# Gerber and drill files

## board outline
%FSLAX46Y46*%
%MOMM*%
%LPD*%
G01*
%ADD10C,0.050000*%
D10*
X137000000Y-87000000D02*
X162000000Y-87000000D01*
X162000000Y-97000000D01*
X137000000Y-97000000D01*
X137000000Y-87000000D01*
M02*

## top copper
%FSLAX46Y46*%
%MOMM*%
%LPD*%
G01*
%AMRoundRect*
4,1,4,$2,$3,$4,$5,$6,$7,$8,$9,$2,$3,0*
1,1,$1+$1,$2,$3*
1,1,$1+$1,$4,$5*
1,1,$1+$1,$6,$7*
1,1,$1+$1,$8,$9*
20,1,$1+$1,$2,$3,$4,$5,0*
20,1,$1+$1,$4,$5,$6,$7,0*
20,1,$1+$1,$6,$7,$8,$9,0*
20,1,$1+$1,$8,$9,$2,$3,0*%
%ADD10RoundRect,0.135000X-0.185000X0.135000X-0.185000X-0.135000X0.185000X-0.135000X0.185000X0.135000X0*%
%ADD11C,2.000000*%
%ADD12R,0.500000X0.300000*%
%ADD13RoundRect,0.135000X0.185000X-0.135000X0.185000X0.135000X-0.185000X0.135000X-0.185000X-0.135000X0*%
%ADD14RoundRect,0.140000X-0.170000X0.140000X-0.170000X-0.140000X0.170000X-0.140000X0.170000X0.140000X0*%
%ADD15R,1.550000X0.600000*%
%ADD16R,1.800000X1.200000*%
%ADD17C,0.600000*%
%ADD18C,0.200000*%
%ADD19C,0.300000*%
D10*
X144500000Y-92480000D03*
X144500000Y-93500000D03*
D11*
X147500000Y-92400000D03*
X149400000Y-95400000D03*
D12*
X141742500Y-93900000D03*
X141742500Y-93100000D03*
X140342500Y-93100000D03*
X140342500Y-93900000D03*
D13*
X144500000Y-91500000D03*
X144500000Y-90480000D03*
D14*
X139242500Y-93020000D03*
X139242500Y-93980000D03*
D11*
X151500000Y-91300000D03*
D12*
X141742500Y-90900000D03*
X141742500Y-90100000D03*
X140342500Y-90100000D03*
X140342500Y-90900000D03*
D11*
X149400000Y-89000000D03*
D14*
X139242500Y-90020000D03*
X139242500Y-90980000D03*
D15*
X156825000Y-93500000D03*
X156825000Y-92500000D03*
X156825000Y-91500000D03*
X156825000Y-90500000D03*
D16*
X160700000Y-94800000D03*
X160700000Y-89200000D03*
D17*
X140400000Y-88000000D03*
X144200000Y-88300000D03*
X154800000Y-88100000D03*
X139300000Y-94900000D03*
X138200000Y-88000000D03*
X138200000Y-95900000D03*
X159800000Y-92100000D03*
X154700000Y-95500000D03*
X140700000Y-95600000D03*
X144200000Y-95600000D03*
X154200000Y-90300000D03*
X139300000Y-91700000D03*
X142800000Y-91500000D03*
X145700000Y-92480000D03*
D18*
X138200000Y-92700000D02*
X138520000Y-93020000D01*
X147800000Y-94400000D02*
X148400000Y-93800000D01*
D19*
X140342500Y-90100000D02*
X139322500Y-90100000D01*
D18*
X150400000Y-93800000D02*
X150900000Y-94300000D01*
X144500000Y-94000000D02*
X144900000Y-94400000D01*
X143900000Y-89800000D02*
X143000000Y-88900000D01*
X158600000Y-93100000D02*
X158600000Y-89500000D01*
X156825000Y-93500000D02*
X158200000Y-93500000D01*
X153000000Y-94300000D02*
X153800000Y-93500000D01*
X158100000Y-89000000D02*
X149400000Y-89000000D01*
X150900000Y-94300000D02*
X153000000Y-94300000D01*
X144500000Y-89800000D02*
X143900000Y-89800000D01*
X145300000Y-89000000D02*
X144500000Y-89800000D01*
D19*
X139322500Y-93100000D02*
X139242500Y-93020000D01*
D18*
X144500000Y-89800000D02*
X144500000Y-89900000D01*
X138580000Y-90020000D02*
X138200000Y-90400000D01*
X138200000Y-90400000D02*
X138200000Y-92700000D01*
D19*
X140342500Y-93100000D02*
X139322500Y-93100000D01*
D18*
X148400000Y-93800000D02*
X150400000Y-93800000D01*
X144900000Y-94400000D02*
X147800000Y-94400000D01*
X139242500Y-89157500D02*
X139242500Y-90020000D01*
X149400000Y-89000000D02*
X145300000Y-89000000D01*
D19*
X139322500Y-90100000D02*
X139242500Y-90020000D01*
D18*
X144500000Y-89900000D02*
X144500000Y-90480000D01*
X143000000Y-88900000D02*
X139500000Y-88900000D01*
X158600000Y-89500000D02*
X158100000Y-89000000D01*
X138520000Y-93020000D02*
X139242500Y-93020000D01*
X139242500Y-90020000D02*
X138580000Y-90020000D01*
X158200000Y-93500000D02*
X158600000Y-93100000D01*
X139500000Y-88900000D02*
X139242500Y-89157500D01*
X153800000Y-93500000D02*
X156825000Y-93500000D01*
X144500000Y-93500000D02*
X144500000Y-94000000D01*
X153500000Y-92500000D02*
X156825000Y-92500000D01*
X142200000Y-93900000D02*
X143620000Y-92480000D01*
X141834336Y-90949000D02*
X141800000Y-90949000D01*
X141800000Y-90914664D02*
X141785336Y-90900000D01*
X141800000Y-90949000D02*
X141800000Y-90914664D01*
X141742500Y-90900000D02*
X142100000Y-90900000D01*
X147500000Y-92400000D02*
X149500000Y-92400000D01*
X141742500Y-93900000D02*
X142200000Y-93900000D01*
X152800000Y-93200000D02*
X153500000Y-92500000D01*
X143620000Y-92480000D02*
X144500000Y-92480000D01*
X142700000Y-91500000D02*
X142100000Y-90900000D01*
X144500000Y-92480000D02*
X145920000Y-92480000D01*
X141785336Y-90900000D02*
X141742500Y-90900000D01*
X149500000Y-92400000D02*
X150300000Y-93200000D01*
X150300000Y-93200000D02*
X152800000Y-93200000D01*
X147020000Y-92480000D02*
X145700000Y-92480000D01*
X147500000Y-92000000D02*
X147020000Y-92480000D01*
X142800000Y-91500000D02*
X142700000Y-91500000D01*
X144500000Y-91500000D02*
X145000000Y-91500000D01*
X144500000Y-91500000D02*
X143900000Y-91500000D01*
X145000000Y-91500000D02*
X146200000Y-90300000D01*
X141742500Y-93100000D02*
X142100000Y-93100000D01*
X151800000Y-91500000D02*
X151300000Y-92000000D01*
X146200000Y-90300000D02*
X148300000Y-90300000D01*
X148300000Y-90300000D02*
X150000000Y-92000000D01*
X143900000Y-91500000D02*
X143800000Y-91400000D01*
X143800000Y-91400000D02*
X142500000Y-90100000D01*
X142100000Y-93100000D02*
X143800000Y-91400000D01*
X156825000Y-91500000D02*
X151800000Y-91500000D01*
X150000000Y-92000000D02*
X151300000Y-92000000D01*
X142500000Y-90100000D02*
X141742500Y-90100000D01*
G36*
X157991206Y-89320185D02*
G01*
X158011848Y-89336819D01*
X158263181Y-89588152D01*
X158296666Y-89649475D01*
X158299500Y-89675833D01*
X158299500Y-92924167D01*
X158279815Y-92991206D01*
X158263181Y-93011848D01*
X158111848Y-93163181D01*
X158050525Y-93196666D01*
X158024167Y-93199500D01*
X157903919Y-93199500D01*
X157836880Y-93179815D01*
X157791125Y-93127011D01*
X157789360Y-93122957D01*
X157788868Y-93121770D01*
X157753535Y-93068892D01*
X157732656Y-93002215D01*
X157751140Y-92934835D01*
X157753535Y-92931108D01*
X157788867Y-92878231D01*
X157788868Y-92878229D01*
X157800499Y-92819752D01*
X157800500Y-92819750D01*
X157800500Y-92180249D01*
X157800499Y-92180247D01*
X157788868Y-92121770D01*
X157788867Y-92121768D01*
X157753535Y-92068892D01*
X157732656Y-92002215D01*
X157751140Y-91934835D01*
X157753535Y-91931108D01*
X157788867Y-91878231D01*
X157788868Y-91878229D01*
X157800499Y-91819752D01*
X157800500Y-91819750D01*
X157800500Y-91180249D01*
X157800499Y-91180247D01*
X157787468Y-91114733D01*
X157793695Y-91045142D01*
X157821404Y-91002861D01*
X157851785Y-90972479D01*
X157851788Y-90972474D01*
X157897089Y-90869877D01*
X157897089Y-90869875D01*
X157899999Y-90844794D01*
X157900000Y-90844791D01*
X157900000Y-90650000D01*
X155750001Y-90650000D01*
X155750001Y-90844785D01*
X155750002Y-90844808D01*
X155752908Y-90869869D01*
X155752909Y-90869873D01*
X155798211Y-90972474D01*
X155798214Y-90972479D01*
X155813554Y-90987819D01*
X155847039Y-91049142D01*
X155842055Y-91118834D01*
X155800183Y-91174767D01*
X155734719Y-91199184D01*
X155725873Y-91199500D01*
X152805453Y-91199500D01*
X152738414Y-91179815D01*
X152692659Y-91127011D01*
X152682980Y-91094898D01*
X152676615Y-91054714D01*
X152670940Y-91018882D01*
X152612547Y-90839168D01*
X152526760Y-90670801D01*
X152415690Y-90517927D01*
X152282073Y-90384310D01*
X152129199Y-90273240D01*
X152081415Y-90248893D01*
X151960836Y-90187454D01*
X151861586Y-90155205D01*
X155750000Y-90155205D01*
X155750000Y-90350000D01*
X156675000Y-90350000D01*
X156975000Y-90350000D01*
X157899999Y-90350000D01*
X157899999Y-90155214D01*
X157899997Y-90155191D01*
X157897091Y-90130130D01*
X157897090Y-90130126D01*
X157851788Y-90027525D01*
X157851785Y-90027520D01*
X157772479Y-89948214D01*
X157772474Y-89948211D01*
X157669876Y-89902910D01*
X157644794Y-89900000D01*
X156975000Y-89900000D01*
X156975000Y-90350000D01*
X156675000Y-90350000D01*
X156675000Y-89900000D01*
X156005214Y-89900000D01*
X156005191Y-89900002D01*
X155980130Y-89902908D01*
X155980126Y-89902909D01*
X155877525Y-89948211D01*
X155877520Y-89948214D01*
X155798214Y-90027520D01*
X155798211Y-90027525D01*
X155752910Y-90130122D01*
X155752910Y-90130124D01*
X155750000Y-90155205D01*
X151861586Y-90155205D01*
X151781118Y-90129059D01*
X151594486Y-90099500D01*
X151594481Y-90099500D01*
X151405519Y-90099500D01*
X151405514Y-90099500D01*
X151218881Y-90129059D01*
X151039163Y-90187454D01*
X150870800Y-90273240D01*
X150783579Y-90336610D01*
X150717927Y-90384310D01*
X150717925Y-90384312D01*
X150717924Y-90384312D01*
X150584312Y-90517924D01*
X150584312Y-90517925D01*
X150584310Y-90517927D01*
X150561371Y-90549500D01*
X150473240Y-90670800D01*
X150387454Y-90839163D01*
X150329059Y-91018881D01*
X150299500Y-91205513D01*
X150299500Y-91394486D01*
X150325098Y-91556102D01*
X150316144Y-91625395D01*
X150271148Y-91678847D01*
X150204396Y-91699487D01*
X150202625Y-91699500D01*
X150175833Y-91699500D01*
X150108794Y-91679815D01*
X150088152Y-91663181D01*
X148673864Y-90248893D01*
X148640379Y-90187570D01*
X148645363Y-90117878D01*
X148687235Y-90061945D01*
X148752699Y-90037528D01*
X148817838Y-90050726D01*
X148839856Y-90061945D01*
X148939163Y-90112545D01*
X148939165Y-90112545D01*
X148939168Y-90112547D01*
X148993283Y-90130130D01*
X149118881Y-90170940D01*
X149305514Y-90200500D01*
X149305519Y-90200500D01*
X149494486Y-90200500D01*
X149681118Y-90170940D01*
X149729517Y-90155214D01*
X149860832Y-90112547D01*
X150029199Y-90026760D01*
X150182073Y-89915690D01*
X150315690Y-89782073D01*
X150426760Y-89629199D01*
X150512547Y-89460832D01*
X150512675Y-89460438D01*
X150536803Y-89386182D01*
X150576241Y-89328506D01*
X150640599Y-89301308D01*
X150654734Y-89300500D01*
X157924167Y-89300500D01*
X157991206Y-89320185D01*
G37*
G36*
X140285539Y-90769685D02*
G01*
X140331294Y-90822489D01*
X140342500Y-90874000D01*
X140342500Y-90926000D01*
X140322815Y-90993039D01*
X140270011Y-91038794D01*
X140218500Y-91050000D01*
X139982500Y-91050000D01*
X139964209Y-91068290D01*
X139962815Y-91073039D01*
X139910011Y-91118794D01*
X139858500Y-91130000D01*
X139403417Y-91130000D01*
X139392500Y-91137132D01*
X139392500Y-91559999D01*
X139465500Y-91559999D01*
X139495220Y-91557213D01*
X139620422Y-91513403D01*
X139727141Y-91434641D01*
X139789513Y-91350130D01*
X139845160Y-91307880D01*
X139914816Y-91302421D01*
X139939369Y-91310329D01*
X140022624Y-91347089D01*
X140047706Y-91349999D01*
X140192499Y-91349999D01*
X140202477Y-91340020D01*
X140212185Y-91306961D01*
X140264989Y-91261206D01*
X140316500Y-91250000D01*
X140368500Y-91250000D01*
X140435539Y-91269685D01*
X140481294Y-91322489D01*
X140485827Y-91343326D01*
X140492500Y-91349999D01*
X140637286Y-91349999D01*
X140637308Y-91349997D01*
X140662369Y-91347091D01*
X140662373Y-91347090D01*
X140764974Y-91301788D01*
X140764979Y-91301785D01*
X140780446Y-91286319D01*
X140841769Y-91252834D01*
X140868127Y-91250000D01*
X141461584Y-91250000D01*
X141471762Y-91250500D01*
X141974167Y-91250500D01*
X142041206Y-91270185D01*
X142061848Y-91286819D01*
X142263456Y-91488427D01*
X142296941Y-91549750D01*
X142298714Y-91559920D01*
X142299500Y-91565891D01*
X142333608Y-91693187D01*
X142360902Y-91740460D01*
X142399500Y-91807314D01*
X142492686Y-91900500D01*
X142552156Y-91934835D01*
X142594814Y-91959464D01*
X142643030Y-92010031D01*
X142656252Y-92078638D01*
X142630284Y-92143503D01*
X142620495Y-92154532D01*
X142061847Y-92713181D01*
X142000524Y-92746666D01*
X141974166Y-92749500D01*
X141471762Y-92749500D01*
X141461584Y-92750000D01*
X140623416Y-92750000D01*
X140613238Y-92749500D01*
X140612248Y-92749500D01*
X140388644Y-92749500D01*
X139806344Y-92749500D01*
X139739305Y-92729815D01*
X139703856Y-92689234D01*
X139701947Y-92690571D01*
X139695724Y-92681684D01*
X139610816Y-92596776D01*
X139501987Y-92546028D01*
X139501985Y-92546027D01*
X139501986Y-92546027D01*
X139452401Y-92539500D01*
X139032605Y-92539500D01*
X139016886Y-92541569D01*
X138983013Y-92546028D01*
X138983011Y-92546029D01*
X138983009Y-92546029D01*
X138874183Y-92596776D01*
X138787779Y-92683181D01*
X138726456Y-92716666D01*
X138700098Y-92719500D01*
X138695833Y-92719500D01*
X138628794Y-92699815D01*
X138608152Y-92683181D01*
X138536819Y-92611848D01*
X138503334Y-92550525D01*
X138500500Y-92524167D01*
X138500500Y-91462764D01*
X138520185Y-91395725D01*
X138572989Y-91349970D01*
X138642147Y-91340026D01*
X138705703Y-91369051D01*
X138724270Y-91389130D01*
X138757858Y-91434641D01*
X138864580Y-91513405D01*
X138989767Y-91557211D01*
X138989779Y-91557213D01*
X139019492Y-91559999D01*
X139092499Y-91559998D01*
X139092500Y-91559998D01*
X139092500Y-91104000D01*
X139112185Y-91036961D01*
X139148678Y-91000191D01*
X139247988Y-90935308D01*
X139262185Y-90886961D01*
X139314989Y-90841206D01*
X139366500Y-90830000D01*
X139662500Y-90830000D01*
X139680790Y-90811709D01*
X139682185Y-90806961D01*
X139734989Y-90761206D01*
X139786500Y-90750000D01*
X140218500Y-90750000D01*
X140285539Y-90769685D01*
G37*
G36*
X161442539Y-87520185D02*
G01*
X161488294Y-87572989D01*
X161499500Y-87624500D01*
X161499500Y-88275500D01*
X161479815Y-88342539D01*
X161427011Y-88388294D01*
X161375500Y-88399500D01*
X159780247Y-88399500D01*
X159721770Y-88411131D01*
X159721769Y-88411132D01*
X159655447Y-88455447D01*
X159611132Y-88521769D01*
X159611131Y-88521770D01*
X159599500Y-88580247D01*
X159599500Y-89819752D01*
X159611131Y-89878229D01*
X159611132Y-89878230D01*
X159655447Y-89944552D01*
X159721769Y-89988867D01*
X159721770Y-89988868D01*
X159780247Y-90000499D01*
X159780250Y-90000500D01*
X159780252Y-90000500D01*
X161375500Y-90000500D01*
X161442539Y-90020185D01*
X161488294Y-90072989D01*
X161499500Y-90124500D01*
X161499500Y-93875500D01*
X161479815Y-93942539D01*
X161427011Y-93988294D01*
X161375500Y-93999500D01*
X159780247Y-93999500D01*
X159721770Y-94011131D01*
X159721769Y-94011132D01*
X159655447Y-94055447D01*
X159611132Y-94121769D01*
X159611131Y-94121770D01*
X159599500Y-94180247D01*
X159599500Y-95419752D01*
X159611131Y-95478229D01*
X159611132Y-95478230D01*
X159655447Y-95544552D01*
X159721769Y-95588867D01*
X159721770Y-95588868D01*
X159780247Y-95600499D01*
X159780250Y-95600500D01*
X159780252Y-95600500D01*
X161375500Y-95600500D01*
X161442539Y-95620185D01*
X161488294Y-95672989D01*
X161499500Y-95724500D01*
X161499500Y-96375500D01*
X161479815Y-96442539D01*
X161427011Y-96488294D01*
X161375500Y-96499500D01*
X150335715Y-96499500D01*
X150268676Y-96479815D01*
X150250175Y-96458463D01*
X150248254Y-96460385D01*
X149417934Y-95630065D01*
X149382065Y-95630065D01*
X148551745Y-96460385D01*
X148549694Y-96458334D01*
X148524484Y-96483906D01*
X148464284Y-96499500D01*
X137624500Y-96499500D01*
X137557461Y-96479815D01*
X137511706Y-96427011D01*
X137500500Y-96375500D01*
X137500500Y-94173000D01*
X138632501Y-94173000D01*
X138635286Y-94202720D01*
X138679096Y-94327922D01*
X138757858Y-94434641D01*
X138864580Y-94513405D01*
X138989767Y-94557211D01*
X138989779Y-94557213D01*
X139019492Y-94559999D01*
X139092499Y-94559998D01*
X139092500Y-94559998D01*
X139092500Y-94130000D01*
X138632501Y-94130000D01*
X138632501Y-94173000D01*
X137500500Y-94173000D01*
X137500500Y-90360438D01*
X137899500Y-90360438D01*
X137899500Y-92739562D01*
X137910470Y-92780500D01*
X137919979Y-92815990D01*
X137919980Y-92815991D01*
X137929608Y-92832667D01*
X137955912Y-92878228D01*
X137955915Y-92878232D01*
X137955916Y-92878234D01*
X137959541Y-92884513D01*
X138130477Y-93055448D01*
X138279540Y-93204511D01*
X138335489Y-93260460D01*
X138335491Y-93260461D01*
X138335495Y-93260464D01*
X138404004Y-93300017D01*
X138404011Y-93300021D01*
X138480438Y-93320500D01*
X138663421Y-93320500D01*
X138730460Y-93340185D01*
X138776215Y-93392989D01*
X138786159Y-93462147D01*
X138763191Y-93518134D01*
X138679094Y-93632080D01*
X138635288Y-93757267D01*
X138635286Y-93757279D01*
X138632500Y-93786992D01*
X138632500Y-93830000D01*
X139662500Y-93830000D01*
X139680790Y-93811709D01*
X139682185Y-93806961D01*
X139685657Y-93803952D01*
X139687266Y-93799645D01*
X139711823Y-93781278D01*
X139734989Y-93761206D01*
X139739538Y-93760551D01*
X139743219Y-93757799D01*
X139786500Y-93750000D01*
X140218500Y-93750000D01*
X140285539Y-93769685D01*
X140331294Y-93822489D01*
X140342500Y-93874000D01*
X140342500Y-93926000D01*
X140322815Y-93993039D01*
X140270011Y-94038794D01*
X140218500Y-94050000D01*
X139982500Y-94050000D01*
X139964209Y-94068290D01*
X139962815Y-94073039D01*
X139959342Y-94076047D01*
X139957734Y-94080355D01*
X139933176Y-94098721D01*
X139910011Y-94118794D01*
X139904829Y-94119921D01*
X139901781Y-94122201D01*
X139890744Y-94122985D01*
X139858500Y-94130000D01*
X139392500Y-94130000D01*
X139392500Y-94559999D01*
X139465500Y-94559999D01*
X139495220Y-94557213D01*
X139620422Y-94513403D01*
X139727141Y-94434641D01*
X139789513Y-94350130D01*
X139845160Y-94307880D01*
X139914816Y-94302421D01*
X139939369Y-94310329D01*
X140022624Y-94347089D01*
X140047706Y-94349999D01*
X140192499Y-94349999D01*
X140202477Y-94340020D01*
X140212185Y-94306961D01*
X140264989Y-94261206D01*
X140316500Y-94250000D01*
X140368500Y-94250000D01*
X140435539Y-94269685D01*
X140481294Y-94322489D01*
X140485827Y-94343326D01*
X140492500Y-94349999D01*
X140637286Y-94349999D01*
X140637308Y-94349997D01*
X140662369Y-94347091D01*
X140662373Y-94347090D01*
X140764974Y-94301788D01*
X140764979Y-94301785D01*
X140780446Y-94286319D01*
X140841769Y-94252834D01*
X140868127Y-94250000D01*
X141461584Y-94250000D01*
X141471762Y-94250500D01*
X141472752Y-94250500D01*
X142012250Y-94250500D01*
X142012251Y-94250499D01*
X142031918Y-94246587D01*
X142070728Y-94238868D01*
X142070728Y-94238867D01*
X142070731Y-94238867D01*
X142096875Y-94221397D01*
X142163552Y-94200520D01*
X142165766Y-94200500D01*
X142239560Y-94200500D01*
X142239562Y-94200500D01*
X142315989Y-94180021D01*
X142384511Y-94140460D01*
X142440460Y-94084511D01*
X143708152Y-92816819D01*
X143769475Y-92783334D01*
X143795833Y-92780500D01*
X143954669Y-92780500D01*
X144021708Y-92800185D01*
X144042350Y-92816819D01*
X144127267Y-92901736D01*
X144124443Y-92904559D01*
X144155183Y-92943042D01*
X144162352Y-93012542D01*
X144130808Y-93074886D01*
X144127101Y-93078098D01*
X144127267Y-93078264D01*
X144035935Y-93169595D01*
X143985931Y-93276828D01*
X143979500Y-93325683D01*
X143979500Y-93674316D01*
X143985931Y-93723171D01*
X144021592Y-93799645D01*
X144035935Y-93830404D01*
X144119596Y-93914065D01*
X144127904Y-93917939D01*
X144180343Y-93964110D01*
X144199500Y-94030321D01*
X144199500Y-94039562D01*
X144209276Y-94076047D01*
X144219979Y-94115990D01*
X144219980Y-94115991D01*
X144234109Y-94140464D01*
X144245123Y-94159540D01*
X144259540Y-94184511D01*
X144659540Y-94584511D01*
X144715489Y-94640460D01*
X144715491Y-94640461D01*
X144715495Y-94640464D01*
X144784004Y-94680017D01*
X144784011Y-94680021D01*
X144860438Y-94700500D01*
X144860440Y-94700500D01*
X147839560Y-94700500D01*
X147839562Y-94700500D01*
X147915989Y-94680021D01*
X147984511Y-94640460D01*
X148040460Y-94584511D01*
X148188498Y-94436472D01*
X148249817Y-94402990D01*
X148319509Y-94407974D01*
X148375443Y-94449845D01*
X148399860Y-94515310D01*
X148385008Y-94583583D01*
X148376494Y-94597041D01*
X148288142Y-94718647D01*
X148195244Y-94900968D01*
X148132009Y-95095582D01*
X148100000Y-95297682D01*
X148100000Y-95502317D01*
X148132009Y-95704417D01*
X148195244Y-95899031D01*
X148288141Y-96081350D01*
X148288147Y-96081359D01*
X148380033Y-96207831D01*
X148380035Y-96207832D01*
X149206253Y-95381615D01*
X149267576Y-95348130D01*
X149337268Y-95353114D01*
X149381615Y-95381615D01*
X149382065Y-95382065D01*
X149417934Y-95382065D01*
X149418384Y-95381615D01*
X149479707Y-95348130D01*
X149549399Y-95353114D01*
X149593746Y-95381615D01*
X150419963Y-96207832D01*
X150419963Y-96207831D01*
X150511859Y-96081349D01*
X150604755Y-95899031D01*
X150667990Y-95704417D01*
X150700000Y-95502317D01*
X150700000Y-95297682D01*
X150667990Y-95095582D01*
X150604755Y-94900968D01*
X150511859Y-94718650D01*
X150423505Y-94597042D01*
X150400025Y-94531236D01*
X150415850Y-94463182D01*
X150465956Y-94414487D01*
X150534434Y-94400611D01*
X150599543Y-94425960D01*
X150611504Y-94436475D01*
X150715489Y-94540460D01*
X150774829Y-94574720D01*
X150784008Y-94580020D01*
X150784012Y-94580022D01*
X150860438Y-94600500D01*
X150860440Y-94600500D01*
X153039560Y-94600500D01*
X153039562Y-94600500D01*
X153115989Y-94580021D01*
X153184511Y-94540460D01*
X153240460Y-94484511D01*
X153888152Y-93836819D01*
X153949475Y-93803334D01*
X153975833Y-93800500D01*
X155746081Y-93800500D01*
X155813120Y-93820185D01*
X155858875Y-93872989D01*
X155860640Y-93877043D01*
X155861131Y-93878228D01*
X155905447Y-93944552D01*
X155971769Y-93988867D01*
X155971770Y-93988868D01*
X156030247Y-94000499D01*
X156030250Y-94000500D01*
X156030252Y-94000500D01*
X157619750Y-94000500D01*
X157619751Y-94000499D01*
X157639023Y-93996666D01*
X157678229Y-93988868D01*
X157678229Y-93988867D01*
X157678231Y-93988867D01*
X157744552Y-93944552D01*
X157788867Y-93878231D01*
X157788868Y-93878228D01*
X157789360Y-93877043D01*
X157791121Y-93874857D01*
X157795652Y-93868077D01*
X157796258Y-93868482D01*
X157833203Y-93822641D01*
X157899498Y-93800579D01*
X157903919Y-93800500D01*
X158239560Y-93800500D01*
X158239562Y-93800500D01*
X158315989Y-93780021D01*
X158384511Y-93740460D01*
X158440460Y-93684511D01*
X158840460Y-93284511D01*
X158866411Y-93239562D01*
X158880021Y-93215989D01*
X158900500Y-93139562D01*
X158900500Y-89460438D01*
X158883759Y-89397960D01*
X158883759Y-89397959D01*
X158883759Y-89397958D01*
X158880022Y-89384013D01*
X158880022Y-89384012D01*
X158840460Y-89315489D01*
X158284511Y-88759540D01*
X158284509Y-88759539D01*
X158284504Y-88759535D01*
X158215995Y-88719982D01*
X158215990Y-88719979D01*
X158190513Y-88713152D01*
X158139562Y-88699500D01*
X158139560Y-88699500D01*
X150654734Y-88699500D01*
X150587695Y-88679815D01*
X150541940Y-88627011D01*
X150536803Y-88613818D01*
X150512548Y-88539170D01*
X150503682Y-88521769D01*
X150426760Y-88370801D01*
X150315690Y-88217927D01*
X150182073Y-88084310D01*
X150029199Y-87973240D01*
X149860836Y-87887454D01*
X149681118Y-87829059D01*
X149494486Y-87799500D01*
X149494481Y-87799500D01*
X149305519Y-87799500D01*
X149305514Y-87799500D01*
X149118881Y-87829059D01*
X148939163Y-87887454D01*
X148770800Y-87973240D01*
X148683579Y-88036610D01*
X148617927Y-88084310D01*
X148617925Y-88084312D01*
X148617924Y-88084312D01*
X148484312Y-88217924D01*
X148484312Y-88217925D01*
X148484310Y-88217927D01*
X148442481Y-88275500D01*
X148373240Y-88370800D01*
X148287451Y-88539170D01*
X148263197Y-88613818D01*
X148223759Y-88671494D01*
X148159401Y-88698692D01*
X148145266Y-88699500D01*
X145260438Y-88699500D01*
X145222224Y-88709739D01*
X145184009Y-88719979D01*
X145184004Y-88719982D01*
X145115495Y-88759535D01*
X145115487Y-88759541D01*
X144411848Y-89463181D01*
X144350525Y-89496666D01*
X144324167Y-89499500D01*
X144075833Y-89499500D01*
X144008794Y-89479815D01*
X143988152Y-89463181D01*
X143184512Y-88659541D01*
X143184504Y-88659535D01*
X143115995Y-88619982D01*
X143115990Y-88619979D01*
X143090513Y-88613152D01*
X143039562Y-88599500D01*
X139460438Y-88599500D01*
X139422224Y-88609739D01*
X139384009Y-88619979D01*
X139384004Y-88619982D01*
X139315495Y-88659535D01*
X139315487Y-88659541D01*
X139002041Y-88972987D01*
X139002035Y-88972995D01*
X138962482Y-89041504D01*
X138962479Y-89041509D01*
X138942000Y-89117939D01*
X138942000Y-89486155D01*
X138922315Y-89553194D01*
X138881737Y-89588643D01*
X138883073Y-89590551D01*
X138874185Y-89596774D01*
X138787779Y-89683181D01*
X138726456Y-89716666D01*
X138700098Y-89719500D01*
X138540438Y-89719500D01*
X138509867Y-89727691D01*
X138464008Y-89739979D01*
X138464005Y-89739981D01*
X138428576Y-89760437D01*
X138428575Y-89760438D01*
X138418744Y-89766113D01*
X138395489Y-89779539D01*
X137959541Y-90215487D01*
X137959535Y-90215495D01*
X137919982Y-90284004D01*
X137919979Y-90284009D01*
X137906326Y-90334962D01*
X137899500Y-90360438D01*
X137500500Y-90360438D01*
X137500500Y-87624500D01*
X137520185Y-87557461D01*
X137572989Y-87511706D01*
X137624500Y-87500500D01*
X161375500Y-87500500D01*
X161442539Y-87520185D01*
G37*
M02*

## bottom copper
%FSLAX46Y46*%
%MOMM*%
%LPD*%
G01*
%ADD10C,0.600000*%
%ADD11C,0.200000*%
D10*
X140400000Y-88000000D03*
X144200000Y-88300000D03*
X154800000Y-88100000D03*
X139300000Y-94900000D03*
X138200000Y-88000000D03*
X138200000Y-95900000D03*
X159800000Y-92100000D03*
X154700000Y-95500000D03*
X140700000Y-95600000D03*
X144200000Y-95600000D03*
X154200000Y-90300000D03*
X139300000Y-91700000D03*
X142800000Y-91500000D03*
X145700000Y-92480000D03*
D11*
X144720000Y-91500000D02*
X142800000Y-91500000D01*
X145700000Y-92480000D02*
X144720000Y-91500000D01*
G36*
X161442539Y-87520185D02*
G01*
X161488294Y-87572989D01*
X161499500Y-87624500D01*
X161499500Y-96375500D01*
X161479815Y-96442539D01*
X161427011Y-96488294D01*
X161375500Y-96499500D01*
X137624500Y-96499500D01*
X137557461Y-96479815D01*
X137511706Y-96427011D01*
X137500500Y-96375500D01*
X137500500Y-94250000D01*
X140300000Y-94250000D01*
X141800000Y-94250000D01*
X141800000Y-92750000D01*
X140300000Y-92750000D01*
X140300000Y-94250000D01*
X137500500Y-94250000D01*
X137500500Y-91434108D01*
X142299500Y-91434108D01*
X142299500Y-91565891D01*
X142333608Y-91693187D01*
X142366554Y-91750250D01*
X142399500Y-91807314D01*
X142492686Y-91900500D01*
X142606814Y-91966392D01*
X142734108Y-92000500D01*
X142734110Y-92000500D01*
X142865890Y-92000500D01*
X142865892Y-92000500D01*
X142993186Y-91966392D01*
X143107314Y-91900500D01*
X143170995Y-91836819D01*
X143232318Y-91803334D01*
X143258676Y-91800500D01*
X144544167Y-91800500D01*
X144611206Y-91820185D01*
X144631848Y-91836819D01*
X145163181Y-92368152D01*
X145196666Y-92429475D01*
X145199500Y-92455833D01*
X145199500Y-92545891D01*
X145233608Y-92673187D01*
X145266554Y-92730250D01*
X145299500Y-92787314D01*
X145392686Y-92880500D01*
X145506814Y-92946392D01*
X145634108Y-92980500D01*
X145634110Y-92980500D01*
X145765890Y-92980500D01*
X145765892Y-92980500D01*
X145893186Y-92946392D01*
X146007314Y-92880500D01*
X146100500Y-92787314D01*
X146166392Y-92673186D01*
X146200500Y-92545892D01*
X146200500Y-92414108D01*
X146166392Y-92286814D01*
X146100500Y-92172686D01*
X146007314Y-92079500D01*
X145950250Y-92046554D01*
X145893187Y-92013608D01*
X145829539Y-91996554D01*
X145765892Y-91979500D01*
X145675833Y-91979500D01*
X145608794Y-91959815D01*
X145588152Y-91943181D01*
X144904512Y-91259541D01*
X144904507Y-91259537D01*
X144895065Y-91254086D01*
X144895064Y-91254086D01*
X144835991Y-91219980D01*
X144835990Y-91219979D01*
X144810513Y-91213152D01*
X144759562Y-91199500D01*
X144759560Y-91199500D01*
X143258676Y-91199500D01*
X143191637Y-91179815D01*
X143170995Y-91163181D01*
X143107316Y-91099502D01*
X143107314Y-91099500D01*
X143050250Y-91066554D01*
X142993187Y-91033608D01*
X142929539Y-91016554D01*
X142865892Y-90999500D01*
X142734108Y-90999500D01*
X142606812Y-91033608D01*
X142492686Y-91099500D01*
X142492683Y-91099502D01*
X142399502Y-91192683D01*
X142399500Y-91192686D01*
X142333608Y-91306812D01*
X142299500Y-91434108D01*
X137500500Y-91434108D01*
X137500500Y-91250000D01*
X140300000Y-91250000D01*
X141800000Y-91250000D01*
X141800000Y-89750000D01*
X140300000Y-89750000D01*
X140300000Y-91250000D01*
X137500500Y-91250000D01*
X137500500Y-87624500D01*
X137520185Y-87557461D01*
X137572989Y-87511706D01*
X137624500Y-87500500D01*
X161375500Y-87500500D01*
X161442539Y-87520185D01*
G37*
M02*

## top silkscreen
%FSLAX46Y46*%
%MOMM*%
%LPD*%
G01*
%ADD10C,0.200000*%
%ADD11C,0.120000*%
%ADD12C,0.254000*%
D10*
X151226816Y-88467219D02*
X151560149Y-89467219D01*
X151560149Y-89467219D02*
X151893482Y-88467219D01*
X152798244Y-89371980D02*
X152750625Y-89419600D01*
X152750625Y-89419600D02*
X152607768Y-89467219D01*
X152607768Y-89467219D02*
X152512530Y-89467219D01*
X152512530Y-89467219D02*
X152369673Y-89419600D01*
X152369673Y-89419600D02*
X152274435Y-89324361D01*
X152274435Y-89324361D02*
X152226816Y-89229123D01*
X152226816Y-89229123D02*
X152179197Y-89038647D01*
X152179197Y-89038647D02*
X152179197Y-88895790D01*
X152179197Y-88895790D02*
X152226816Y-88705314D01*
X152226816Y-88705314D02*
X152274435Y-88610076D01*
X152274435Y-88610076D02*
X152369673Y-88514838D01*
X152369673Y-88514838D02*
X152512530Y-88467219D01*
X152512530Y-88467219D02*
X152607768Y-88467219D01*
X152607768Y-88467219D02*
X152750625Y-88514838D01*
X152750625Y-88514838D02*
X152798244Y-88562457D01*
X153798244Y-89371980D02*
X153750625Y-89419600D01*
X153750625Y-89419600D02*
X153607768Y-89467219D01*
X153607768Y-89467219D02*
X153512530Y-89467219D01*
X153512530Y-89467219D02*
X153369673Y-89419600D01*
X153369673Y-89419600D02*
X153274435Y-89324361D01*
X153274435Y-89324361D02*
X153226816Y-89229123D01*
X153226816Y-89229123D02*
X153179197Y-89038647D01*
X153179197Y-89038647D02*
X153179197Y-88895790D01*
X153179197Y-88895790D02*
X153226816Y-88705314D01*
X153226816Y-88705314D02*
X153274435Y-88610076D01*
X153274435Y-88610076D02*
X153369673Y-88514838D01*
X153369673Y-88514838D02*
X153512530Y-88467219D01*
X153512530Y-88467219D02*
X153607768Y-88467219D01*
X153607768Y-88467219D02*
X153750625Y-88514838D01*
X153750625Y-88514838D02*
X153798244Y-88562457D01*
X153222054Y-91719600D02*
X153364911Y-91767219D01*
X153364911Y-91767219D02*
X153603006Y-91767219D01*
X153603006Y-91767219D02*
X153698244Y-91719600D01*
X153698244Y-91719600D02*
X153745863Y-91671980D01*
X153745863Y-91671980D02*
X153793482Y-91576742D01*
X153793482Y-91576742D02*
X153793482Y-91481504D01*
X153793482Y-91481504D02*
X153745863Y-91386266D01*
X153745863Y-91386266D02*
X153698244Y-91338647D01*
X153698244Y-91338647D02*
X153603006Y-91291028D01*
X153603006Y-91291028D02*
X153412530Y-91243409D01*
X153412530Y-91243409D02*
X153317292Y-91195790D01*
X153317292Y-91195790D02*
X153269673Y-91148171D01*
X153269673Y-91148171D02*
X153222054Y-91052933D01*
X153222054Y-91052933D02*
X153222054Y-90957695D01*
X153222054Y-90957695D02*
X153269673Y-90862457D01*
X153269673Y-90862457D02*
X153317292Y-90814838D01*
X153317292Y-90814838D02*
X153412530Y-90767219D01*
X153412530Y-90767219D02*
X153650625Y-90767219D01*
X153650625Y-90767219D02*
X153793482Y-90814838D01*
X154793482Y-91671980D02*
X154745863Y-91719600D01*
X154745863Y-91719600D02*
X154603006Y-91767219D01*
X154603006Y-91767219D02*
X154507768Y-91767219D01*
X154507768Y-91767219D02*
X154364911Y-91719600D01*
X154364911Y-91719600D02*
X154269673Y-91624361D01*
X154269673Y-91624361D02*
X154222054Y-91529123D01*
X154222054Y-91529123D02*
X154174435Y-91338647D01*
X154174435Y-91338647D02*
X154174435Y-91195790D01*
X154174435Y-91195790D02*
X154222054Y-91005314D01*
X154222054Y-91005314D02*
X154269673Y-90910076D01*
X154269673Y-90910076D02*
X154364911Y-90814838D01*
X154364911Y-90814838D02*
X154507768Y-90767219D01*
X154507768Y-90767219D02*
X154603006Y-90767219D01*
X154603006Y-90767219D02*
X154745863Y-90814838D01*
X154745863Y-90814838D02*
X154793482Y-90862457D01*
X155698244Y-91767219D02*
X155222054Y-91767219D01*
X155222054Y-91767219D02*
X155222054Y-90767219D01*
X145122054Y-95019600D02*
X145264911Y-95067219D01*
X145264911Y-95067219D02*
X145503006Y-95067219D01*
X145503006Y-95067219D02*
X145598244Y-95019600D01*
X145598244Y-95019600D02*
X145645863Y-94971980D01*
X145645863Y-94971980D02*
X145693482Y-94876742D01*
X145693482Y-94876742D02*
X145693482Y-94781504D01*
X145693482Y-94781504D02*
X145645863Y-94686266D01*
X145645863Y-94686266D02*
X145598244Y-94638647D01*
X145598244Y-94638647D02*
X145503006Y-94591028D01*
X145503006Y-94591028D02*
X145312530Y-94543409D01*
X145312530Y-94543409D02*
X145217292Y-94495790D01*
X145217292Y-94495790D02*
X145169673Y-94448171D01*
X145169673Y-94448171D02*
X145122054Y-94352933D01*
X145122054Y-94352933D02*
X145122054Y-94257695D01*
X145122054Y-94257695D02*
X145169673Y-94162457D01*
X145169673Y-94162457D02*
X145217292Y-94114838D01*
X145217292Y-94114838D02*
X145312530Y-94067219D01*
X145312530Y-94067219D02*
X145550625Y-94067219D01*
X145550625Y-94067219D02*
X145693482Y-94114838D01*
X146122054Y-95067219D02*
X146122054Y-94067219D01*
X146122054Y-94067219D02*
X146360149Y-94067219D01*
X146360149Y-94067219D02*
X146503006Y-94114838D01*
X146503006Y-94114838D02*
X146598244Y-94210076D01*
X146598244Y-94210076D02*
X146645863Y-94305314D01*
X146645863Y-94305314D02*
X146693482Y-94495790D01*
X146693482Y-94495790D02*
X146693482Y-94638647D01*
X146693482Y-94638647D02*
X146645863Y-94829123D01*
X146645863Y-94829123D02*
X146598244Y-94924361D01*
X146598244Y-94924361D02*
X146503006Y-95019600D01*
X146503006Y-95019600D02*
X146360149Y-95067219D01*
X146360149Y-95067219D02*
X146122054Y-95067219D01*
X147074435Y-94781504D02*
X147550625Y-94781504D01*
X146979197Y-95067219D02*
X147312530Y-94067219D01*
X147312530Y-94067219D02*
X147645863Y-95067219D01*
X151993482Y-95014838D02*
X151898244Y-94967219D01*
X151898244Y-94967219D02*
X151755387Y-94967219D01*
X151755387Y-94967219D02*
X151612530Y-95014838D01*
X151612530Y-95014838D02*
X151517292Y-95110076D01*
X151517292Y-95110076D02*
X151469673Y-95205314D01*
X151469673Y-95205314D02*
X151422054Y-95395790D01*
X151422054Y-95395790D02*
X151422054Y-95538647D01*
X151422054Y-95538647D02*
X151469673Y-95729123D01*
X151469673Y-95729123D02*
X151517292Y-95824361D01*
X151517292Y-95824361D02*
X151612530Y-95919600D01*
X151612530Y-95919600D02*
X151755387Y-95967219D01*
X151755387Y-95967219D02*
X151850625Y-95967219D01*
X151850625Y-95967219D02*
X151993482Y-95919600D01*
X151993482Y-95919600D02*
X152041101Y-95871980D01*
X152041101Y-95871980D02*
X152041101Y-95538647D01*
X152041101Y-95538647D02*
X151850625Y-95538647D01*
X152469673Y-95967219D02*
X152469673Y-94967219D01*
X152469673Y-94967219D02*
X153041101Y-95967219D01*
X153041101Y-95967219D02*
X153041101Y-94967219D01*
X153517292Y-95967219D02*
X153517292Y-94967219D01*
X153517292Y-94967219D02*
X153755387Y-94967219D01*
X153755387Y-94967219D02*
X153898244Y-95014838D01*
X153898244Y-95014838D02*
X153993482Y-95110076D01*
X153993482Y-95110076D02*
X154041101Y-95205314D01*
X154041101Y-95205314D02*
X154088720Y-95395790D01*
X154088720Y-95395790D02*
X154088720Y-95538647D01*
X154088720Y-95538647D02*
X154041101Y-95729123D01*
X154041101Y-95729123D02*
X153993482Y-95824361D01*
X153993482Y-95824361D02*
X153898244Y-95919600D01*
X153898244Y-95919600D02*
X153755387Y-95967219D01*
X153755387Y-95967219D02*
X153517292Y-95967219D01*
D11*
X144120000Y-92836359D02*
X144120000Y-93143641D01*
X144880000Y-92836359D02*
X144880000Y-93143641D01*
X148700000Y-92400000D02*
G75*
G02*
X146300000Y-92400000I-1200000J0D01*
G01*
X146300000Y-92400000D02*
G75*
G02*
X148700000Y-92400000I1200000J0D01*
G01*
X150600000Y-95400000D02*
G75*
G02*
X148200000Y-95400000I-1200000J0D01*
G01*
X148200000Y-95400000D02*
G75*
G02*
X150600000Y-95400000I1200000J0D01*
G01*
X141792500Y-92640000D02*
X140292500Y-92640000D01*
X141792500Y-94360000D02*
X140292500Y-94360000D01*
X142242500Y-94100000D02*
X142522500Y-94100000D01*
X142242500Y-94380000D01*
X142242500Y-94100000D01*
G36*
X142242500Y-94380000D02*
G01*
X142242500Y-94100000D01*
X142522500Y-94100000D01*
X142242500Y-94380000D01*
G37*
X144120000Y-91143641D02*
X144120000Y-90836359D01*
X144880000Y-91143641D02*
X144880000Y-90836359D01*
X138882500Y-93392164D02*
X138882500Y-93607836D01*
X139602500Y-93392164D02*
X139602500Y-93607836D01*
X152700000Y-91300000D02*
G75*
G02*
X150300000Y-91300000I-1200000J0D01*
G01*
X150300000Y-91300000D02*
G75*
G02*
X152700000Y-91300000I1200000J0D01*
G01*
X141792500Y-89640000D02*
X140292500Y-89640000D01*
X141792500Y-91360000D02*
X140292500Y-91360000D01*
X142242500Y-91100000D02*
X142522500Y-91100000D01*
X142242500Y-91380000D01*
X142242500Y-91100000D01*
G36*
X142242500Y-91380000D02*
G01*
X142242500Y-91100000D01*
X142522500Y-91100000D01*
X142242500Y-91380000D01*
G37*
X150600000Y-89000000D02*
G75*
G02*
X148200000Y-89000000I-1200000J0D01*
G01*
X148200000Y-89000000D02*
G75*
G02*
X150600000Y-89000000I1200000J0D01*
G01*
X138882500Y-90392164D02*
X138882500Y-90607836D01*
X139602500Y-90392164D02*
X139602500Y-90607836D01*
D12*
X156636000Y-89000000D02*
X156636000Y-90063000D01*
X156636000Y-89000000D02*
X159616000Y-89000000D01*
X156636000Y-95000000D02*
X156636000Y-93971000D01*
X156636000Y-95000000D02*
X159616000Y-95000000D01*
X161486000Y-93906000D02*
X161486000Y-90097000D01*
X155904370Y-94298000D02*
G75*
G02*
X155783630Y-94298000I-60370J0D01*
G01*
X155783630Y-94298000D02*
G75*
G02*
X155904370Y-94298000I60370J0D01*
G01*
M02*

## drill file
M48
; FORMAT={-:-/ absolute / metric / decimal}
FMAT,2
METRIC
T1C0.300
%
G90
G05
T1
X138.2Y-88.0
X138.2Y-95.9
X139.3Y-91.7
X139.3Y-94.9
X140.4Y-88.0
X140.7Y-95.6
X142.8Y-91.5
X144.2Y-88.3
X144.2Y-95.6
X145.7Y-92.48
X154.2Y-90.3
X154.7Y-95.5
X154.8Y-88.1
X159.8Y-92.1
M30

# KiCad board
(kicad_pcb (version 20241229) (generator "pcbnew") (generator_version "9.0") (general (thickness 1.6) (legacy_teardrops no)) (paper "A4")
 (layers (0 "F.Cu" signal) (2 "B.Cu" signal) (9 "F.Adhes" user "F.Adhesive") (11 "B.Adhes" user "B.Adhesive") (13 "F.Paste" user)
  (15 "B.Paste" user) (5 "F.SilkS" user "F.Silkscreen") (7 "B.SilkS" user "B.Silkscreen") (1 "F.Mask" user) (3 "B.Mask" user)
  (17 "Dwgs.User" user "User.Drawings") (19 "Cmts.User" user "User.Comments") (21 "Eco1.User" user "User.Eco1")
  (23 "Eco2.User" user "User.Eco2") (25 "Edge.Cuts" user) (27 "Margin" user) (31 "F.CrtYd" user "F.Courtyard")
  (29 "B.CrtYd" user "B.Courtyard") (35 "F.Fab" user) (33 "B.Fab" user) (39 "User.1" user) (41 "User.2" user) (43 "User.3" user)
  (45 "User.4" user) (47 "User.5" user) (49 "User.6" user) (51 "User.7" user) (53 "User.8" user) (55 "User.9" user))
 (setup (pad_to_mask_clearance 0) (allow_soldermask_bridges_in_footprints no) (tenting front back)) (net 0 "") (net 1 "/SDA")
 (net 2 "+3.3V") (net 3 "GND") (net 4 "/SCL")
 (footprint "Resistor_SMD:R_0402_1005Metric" (layer "F.Cu") (at 144.5 92.99 -90)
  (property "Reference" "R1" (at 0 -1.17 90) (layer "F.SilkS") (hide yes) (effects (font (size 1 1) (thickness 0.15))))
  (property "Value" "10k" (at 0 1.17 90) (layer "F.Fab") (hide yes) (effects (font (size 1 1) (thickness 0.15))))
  (fp_line (start -0.153641 0.38) (end 0.153641 0.38) (stroke (width 0.12) (type solid)) (layer "F.SilkS"))
  (fp_line (start -0.153641 -0.38) (end 0.153641 -0.38) (stroke (width 0.12) (type solid)) (layer "F.SilkS"))
  (pad "1" smd roundrect (at -0.51 0 270) (size 0.54 0.64) (layers "F.Cu" "F.Mask" "F.Paste") (roundrect_rratio 0.25) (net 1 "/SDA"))
  (pad "2" smd roundrect (at 0.51 0 270) (size 0.54 0.64) (layers "F.Cu" "F.Mask" "F.Paste") (roundrect_rratio 0.25) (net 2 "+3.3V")))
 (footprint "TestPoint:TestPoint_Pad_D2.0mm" (layer "F.Cu") (at 147.5 92.4)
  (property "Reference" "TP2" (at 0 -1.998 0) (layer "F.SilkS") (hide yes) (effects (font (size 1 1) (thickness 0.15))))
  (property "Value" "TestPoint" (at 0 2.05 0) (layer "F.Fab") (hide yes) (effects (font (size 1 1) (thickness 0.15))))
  (fp_circle (center 0 0) (end 0 1.2) (stroke (width 0.12) (type solid)) (fill no) (layer "F.SilkS"))
  (pad "1" smd circle (at 0 0) (size 2 2) (layers "F.Cu" "F.Mask") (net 1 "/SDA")))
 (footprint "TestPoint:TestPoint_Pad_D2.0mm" (layer "F.Cu") (at 149.4 95.4)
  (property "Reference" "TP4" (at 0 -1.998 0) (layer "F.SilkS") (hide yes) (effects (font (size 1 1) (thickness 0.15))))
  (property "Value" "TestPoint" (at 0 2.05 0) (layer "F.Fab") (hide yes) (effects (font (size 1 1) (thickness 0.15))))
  (fp_circle (center 0 0) (end 0 1.2) (stroke (width 0.12) (type solid)) (fill no) (layer "F.SilkS"))
  (pad "1" smd circle (at 0 0) (size 2 2) (layers "F.Cu" "F.Mask") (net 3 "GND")))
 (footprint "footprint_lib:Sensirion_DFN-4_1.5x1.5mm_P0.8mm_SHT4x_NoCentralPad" (layer "F.Cu") (at 141.0425 93.5 180)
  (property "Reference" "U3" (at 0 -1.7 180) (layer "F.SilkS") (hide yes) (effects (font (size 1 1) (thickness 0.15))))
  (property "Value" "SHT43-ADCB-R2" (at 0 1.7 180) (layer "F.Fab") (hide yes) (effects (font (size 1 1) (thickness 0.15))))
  (fp_line (start -0.75 0.86) (end 0.75 0.86) (stroke (width 0.12) (type solid)) (layer "F.SilkS"))
  (fp_line (start -0.75 -0.86) (end 0.75 -0.86) (stroke (width 0.12) (type solid)) (layer "F.SilkS"))
  (fp_poly
   (pts (xy -1.2 -0.6) (xy -1.48 -0.6) (xy -1.2 -0.88) (xy -1.2 -0.6)) (stroke (width 0.12) (type solid)) (fill yes) (layer "F.SilkS"))
  (pad "1" smd rect (at -0.7 -0.4 180) (size 0.5 0.3) (layers "F.Cu" "F.Mask" "F.Paste") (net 1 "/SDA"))
  (pad "2" smd rect (at -0.7 0.4 180) (size 0.5 0.3) (layers "F.Cu" "F.Mask" "F.Paste") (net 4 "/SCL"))
  (pad "3" smd rect (at 0.7 0.4 180) (size 0.5 0.3) (layers "F.Cu" "F.Mask" "F.Paste") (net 2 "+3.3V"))
  (pad "4" smd rect (at 0.7 -0.4 180) (size 0.5 0.3) (layers "F.Cu" "F.Mask" "F.Paste") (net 3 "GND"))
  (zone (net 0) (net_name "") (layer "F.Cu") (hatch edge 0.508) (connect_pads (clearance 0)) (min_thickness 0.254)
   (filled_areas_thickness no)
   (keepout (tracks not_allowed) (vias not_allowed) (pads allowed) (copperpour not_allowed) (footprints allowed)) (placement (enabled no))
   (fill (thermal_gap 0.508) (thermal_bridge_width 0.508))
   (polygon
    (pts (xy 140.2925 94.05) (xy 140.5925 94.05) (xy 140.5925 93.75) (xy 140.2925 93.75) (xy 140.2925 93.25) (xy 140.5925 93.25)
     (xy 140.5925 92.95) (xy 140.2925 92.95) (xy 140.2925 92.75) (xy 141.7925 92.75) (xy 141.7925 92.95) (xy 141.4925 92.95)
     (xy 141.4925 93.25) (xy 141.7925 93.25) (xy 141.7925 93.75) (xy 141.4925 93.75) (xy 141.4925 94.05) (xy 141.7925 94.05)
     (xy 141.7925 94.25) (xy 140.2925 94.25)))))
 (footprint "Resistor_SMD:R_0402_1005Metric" (layer "F.Cu") (at 144.5 90.99 90)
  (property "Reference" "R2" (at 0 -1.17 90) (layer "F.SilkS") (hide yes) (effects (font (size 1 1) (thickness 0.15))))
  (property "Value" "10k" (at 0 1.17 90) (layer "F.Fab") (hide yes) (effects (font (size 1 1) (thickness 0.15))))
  (fp_line (start -0.153641 -0.38) (end 0.153641 -0.38) (stroke (width 0.12) (type solid)) (layer "F.SilkS"))
  (fp_line (start -0.153641 0.38) (end 0.153641 0.38) (stroke (width 0.12) (type solid)) (layer "F.SilkS"))
  (pad "1" smd roundrect (at -0.51 0 90) (size 0.54 0.64) (layers "F.Cu" "F.Mask" "F.Paste") (roundrect_rratio 0.25) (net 4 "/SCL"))
  (pad "2" smd roundrect (at 0.51 0 90) (size 0.54 0.64) (layers "F.Cu" "F.Mask" "F.Paste") (roundrect_rratio 0.25) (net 2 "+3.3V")))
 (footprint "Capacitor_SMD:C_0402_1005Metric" (layer "F.Cu") (at 139.2425 93.5 -90)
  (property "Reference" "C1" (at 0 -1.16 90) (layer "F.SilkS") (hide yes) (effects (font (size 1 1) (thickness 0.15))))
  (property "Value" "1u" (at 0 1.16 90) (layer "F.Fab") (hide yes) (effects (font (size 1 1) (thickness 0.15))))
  (fp_line (start -0.107836 0.36) (end 0.107836 0.36) (stroke (width 0.12) (type solid)) (layer "F.SilkS"))
  (fp_line (start -0.107836 -0.36) (end 0.107836 -0.36) (stroke (width 0.12) (type solid)) (layer "F.SilkS"))
  (pad "1" smd roundrect (at -0.48 0 270) (size 0.56 0.62) (layers "F.Cu" "F.Mask" "F.Paste") (roundrect_rratio 0.25) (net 2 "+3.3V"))
  (pad "2" smd roundrect (at 0.48 0 270) (size 0.56 0.62) (layers "F.Cu" "F.Mask" "F.Paste") (roundrect_rratio 0.25) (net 3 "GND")))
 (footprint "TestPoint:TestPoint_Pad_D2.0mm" (layer "F.Cu") (at 151.5 91.3)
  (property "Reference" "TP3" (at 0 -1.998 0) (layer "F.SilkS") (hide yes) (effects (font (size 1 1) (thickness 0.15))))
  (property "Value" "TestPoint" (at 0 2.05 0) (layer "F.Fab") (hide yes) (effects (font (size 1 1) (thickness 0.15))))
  (fp_circle (center 0 0) (end 0 1.2) (stroke (width 0.12) (type solid)) (fill no) (layer "F.SilkS"))
  (pad "1" smd circle (at 0 0) (size 2 2) (layers "F.Cu" "F.Mask") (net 4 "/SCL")))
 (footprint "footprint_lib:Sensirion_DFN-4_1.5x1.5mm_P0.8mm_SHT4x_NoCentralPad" (layer "F.Cu") (at 141.0425 90.5 180)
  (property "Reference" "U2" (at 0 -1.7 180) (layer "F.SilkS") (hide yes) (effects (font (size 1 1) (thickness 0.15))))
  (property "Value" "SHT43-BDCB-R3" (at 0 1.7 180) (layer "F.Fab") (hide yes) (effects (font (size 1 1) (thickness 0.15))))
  (fp_line (start -0.75 0.86) (end 0.75 0.86) (stroke (width 0.12) (type solid)) (layer "F.SilkS"))
  (fp_line (start -0.75 -0.86) (end 0.75 -0.86) (stroke (width 0.12) (type solid)) (layer "F.SilkS"))
  (fp_poly
   (pts (xy -1.2 -0.6) (xy -1.48 -0.6) (xy -1.2 -0.88) (xy -1.2 -0.6)) (stroke (width 0.12) (type solid)) (fill yes) (layer "F.SilkS"))
  (pad "1" smd rect (at -0.7 -0.4 180) (size 0.5 0.3) (layers "F.Cu" "F.Mask" "F.Paste") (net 1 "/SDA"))
  (pad "2" smd rect (at -0.7 0.4 180) (size 0.5 0.3) (layers "F.Cu" "F.Mask" "F.Paste") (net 4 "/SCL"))
  (pad "3" smd rect (at 0.7 0.4 180) (size 0.5 0.3) (layers "F.Cu" "F.Mask" "F.Paste") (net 2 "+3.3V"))
  (pad "4" smd rect (at 0.7 -0.4 180) (size 0.5 0.3) (layers "F.Cu" "F.Mask" "F.Paste") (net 3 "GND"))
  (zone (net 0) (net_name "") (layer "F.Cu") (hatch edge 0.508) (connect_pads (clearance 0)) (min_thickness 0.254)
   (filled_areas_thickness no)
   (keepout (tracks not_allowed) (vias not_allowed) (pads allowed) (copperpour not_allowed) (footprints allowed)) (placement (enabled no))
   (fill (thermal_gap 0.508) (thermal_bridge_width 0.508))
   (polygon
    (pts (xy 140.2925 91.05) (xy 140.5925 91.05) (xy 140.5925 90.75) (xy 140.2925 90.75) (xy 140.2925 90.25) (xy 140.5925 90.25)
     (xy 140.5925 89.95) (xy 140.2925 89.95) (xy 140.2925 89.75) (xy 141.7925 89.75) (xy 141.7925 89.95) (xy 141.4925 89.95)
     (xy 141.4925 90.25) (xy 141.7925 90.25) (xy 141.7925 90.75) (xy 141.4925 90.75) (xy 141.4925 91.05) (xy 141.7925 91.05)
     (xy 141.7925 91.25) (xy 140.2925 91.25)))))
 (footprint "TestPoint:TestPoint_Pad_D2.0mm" (layer "F.Cu") (at 149.4 89)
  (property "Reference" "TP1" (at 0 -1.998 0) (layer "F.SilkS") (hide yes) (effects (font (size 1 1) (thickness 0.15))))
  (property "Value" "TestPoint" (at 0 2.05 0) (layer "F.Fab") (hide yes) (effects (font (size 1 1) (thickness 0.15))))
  (fp_circle (center 0 0) (end 0 1.2) (stroke (width 0.12) (type solid)) (fill no) (layer "F.SilkS"))
  (pad "1" smd circle (at 0 0) (size 2 2) (layers "F.Cu" "F.Mask") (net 2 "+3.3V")))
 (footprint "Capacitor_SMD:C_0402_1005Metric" (layer "F.Cu") (at 139.2425 90.5 -90)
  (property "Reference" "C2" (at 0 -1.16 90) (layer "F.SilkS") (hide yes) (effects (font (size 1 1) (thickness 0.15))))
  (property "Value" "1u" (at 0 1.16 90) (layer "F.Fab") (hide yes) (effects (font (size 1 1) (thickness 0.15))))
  (fp_line (start -0.107836 0.36) (end 0.107836 0.36) (stroke (width 0.12) (type solid)) (layer "F.SilkS"))
  (fp_line (start -0.107836 -0.36) (end 0.107836 -0.36) (stroke (width 0.12) (type solid)) (layer "F.SilkS"))
  (pad "1" smd roundrect (at -0.48 0 270) (size 0.56 0.62) (layers "F.Cu" "F.Mask" "F.Paste") (roundrect_rratio 0.25) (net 2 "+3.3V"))
  (pad "2" smd roundrect (at 0.48 0 270) (size 0.56 0.62) (layers "F.Cu" "F.Mask" "F.Paste") (roundrect_rratio 0.25) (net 3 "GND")))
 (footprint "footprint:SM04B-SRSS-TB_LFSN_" (layer "F.Cu") (at 161.486 95 90)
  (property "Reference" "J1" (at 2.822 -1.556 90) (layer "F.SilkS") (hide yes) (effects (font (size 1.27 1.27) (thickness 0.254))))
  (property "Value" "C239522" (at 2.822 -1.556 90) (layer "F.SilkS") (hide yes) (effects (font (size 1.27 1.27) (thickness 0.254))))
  (fp_line (start 6 -4.85) (end 4.937 -4.85) (stroke (width 0.254) (type solid)) (layer "F.SilkS"))
  (fp_line (start 6 -4.85) (end 6 -1.87) (stroke (width 0.254) (type solid)) (layer "F.SilkS"))
  (fp_line (start 0 -4.85) (end 1.029 -4.85) (stroke (width 0.254) (type solid)) (layer "F.SilkS"))
  (fp_line (start 0 -4.85) (end 0 -1.87) (stroke (width 0.254) (type solid)) (layer "F.SilkS"))
  (fp_line (start 1.094 0) (end 4.903 0) (stroke (width 0.254) (type solid)) (layer "F.SilkS"))
  (fp_circle (center 0.702 -5.642) (end 0.702 -5.58163) (stroke (width 0.254) (type solid)) (fill no) (layer "F.SilkS"))
  (pad "1" smd rect (at 1.5 -4.661 90) (size 0.6 1.55) (layers "F.Cu" "F.Mask" "F.Paste") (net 2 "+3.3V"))
  (pad "2" smd rect (at 2.5 -4.661 90) (size 0.6 1.55) (layers "F.Cu" "F.Mask" "F.Paste") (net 1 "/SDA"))
  (pad "3" smd rect (at 3.5 -4.661 90) (size 0.6 1.55) (layers "F.Cu" "F.Mask" "F.Paste") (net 4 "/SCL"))
  (pad "4" smd rect (at 4.5 -4.661 90) (size 0.6 1.55) (layers "F.Cu" "F.Mask" "F.Paste") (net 3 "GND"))
  (pad "5" smd rect (at 0.2 -0.786 90) (size 1.2 1.8) (layers "F.Cu" "F.Mask" "F.Paste"))
  (pad "6" smd rect (at 5.8 -0.786 90) (size 1.2 1.8) (layers "F.Cu" "F.Mask" "F.Paste")))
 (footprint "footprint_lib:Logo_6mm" (layer "B.Cu") (at 152.2 91.8 180)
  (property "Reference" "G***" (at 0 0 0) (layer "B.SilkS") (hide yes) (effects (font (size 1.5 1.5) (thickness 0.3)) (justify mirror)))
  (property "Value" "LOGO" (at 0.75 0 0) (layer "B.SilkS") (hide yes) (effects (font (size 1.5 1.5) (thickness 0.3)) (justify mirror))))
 (gr_rect (start 137 87) (end 162 97) (stroke (width 0.05) (type default)) (fill no) (layer "Edge.Cuts"))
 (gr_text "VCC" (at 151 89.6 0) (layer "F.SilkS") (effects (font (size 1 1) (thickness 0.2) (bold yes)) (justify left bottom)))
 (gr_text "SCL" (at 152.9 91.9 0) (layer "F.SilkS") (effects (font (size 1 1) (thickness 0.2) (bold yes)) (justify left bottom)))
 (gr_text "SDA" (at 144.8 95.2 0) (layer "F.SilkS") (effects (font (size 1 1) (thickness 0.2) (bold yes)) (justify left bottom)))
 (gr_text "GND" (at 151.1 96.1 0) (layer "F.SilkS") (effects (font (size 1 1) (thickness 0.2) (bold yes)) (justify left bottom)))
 (segment (start 138.2 92.7) (end 138.52 93.02) (width 0.2) (layer "F.Cu") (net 2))
 (segment (start 147.8 94.4) (end 148.4 93.8) (width 0.2) (layer "F.Cu") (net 2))
 (segment (start 140.3425 90.1) (end 139.3225 90.1) (width 0.3) (layer "F.Cu") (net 2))
 (segment (start 150.4 93.8) (end 150.9 94.3) (width 0.2) (layer "F.Cu") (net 2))
 (segment (start 144.5 94) (end 144.9 94.4) (width 0.2) (layer "F.Cu") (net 2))
 (segment (start 143.9 89.8) (end 143 88.9) (width 0.2) (layer "F.Cu") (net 2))
 (segment (start 158.6 93.1) (end 158.6 89.5) (width 0.2) (layer "F.Cu") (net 2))
 (segment (start 156.825 93.5) (end 158.2 93.5) (width 0.2) (layer "F.Cu") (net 2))
 (segment (start 153 94.3) (end 153.8 93.5) (width 0.2) (layer "F.Cu") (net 2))
 (segment (start 158.1 89) (end 149.4 89) (width 0.2) (layer "F.Cu") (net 2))
 (segment (start 150.9 94.3) (end 153 94.3) (width 0.2) (layer "F.Cu") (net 2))
 (segment (start 144.5 89.8) (end 143.9 89.8) (width 0.2) (layer "F.Cu") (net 2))
 (segment (start 145.3 89) (end 144.5 89.8) (width 0.2) (layer "F.Cu") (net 2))
 (segment (start 139.3225 93.1) (end 139.2425 93.02) (width 0.3) (layer "F.Cu") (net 2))
 (segment (start 144.5 89.8) (end 144.5 89.9) (width 0.2) (layer "F.Cu") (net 2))
 (segment (start 138.58 90.02) (end 138.2 90.4) (width 0.2) (layer "F.Cu") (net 2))
 (segment (start 138.2 90.4) (end 138.2 92.7) (width 0.2) (layer "F.Cu") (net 2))
 (segment (start 140.3425 93.1) (end 139.3225 93.1) (width 0.3) (layer "F.Cu") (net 2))
 (segment (start 148.4 93.8) (end 150.4 93.8) (width 0.2) (layer "F.Cu") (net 2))
 (segment (start 144.9 94.4) (end 147.8 94.4) (width 0.2) (layer "F.Cu") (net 2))
 (segment (start 139.2425 89.1575) (end 139.2425 90.02) (width 0.2) (layer "F.Cu") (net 2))
 (segment (start 149.4 89) (end 145.3 89) (width 0.2) (layer "F.Cu") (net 2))
 (segment (start 139.3225 90.1) (end 139.2425 90.02) (width 0.3) (layer "F.Cu") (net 2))
 (segment (start 144.5 89.9) (end 144.5 90.48) (width 0.2) (layer "F.Cu") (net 2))
 (segment (start 143 88.9) (end 139.5 88.9) (width 0.2) (layer "F.Cu") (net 2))
 (segment (start 158.6 89.5) (end 158.1 89) (width 0.2) (layer "F.Cu") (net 2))
 (segment (start 138.52 93.02) (end 139.2425 93.02) (width 0.2) (layer "F.Cu") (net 2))
 (segment (start 139.2425 90.02) (end 138.58 90.02) (width 0.2) (layer "F.Cu") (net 2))
 (segment (start 158.2 93.5) (end 158.6 93.1) (width 0.2) (layer "F.Cu") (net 2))
 (segment (start 139.5 88.9) (end 139.2425 89.1575) (width 0.2) (layer "F.Cu") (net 2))
 (segment (start 153.8 93.5) (end 156.825 93.5) (width 0.2) (layer "F.Cu") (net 2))
 (segment (start 144.5 93.5) (end 144.5 94) (width 0.2) (layer "F.Cu") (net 2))
 (via (at 140.4 88) (size 0.6) (drill 0.3) (layers "F.Cu" "B.Cu") (free yes) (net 3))
 (via (at 144.2 88.3) (size 0.6) (drill 0.3) (layers "F.Cu" "B.Cu") (free yes) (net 3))
 (via (at 154.8 88.1) (size 0.6) (drill 0.3) (layers "F.Cu" "B.Cu") (free yes) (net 3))
 (via (at 139.3 94.9) (size 0.6) (drill 0.3) (layers "F.Cu" "B.Cu") (free yes) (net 3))
 (via (at 138.2 88) (size 0.6) (drill 0.3) (layers "F.Cu" "B.Cu") (free yes) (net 3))
 (via (at 138.2 95.9) (size 0.6) (drill 0.3) (layers "F.Cu" "B.Cu") (free yes) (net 3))
 (via (at 159.8 92.1) (size 0.6) (drill 0.3) (layers "F.Cu" "B.Cu") (free yes) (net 3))
 (via (at 154.7 95.5) (size 0.6) (drill 0.3) (layers "F.Cu" "B.Cu") (free yes) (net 3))
 (via (at 140.7 95.6) (size 0.6) (drill 0.3) (layers "F.Cu" "B.Cu") (free yes) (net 3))
 (via (at 144.2 95.6) (size 0.6) (drill 0.3) (layers "F.Cu" "B.Cu") (free yes) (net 3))
 (via (at 154.2 90.3) (size 0.6) (drill 0.3) (layers "F.Cu" "B.Cu") (free yes) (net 3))
 (via (at 139.3 91.7) (size 0.6) (drill 0.3) (layers "F.Cu" "B.Cu") (free yes) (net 3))
 (segment (start 153.5 92.5) (end 156.825 92.5) (width 0.2) (layer "F.Cu") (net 1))
 (segment (start 142.2 93.9) (end 143.62 92.48) (width 0.2) (layer "F.Cu") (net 1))
 (segment (start 141.834336 90.949) (end 141.8 90.949) (width 0.2) (layer "F.Cu") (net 1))
 (segment (start 141.8 90.914664) (end 141.785336 90.9) (width 0.2) (layer "F.Cu") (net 1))
 (segment (start 141.8 90.949) (end 141.8 90.914664) (width 0.2) (layer "F.Cu") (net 1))
 (segment (start 141.7425 90.9) (end 142.1 90.9) (width 0.2) (layer "F.Cu") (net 1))
 (segment (start 147.5 92.4) (end 149.5 92.4) (width 0.2) (layer "F.Cu") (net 1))
 (segment (start 141.7425 93.9) (end 142.2 93.9) (width 0.2) (layer "F.Cu") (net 1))
 (segment (start 152.8 93.2) (end 153.5 92.5) (width 0.2) (layer "F.Cu") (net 1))
 (segment (start 143.62 92.48) (end 144.5 92.48) (width 0.2) (layer "F.Cu") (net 1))
 (segment (start 142.7 91.5) (end 142.1 90.9) (width 0.2) (layer "F.Cu") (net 1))
 (segment (start 144.5 92.48) (end 145.92 92.48) (width 0.2) (layer "F.Cu") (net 1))
 (segment (start 141.785336 90.9) (end 141.7425 90.9) (width 0.2) (layer "F.Cu") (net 1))
 (segment (start 149.5 92.4) (end 150.3 93.2) (width 0.2) (layer "F.Cu") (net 1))
 (segment (start 150.3 93.2) (end 152.8 93.2) (width 0.2) (layer "F.Cu") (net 1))
 (segment (start 147.02 92.48) (end 145.7 92.48) (width 0.2) (layer "F.Cu") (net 1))
 (segment (start 147.5 92) (end 147.02 92.48) (width 0.2) (layer "F.Cu") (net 1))
 (segment (start 142.8 91.5) (end 142.7 91.5) (width 0.2) (layer "F.Cu") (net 1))
 (via (at 142.8 91.5) (size 0.6) (drill 0.3) (layers "F.Cu" "B.Cu") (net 1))
 (via (at 145.7 92.48) (size 0.6) (drill 0.3) (layers "F.Cu" "B.Cu") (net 1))
 (segment (start 144.72 91.5) (end 142.8 91.5) (width 0.2) (layer "B.Cu") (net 1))
 (segment (start 145.7 92.48) (end 144.72 91.5) (width 0.2) (layer "B.Cu") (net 1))
 (segment (start 144.5 91.5) (end 145 91.5) (width 0.2) (layer "F.Cu") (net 4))
 (segment (start 144.5 91.5) (end 143.9 91.5) (width 0.2) (layer "F.Cu") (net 4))
 (segment (start 145 91.5) (end 146.2 90.3) (width 0.2) (layer "F.Cu") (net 4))
 (segment (start 141.7425 93.1) (end 142.1 93.1) (width 0.2) (layer "F.Cu") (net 4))
 (segment (start 151.8 91.5) (end 151.3 92) (width 0.2) (layer "F.Cu") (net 4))
 (segment (start 146.2 90.3) (end 148.3 90.3) (width 0.2) (layer "F.Cu") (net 4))
 (segment (start 148.3 90.3) (end 150 92) (width 0.2) (layer "F.Cu") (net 4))
 (segment (start 143.9 91.5) (end 143.8 91.4) (width 0.2) (layer "F.Cu") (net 4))
 (segment (start 143.8 91.4) (end 142.5 90.1) (width 0.2) (layer "F.Cu") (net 4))
 (segment (start 142.1 93.1) (end 143.8 91.4) (width 0.2) (layer "F.Cu") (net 4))
 (segment (start 156.825 91.5) (end 151.8 91.5) (width 0.2) (layer "F.Cu") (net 4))
 (segment (start 150 92) (end 151.3 92) (width 0.2) (layer "F.Cu") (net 4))
 (segment (start 142.5 90.1) (end 141.7425 90.1) (width 0.2) (layer "F.Cu") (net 4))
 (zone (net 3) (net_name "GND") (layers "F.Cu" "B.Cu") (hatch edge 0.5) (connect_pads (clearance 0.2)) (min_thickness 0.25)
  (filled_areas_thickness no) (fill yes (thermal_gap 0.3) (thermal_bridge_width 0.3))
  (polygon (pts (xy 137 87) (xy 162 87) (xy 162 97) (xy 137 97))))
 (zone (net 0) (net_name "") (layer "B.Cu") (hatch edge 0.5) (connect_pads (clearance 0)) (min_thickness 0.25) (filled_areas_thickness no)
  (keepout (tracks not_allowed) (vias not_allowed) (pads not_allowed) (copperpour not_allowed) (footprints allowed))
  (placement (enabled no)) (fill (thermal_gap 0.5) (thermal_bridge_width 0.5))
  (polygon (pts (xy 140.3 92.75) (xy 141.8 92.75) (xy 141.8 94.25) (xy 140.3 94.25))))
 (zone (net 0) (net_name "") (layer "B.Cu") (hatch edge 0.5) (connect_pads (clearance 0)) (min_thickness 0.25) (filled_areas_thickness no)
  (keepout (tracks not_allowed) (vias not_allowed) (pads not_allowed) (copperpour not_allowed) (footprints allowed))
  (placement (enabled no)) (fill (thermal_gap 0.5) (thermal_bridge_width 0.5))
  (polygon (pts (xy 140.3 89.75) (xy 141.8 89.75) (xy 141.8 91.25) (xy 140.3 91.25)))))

